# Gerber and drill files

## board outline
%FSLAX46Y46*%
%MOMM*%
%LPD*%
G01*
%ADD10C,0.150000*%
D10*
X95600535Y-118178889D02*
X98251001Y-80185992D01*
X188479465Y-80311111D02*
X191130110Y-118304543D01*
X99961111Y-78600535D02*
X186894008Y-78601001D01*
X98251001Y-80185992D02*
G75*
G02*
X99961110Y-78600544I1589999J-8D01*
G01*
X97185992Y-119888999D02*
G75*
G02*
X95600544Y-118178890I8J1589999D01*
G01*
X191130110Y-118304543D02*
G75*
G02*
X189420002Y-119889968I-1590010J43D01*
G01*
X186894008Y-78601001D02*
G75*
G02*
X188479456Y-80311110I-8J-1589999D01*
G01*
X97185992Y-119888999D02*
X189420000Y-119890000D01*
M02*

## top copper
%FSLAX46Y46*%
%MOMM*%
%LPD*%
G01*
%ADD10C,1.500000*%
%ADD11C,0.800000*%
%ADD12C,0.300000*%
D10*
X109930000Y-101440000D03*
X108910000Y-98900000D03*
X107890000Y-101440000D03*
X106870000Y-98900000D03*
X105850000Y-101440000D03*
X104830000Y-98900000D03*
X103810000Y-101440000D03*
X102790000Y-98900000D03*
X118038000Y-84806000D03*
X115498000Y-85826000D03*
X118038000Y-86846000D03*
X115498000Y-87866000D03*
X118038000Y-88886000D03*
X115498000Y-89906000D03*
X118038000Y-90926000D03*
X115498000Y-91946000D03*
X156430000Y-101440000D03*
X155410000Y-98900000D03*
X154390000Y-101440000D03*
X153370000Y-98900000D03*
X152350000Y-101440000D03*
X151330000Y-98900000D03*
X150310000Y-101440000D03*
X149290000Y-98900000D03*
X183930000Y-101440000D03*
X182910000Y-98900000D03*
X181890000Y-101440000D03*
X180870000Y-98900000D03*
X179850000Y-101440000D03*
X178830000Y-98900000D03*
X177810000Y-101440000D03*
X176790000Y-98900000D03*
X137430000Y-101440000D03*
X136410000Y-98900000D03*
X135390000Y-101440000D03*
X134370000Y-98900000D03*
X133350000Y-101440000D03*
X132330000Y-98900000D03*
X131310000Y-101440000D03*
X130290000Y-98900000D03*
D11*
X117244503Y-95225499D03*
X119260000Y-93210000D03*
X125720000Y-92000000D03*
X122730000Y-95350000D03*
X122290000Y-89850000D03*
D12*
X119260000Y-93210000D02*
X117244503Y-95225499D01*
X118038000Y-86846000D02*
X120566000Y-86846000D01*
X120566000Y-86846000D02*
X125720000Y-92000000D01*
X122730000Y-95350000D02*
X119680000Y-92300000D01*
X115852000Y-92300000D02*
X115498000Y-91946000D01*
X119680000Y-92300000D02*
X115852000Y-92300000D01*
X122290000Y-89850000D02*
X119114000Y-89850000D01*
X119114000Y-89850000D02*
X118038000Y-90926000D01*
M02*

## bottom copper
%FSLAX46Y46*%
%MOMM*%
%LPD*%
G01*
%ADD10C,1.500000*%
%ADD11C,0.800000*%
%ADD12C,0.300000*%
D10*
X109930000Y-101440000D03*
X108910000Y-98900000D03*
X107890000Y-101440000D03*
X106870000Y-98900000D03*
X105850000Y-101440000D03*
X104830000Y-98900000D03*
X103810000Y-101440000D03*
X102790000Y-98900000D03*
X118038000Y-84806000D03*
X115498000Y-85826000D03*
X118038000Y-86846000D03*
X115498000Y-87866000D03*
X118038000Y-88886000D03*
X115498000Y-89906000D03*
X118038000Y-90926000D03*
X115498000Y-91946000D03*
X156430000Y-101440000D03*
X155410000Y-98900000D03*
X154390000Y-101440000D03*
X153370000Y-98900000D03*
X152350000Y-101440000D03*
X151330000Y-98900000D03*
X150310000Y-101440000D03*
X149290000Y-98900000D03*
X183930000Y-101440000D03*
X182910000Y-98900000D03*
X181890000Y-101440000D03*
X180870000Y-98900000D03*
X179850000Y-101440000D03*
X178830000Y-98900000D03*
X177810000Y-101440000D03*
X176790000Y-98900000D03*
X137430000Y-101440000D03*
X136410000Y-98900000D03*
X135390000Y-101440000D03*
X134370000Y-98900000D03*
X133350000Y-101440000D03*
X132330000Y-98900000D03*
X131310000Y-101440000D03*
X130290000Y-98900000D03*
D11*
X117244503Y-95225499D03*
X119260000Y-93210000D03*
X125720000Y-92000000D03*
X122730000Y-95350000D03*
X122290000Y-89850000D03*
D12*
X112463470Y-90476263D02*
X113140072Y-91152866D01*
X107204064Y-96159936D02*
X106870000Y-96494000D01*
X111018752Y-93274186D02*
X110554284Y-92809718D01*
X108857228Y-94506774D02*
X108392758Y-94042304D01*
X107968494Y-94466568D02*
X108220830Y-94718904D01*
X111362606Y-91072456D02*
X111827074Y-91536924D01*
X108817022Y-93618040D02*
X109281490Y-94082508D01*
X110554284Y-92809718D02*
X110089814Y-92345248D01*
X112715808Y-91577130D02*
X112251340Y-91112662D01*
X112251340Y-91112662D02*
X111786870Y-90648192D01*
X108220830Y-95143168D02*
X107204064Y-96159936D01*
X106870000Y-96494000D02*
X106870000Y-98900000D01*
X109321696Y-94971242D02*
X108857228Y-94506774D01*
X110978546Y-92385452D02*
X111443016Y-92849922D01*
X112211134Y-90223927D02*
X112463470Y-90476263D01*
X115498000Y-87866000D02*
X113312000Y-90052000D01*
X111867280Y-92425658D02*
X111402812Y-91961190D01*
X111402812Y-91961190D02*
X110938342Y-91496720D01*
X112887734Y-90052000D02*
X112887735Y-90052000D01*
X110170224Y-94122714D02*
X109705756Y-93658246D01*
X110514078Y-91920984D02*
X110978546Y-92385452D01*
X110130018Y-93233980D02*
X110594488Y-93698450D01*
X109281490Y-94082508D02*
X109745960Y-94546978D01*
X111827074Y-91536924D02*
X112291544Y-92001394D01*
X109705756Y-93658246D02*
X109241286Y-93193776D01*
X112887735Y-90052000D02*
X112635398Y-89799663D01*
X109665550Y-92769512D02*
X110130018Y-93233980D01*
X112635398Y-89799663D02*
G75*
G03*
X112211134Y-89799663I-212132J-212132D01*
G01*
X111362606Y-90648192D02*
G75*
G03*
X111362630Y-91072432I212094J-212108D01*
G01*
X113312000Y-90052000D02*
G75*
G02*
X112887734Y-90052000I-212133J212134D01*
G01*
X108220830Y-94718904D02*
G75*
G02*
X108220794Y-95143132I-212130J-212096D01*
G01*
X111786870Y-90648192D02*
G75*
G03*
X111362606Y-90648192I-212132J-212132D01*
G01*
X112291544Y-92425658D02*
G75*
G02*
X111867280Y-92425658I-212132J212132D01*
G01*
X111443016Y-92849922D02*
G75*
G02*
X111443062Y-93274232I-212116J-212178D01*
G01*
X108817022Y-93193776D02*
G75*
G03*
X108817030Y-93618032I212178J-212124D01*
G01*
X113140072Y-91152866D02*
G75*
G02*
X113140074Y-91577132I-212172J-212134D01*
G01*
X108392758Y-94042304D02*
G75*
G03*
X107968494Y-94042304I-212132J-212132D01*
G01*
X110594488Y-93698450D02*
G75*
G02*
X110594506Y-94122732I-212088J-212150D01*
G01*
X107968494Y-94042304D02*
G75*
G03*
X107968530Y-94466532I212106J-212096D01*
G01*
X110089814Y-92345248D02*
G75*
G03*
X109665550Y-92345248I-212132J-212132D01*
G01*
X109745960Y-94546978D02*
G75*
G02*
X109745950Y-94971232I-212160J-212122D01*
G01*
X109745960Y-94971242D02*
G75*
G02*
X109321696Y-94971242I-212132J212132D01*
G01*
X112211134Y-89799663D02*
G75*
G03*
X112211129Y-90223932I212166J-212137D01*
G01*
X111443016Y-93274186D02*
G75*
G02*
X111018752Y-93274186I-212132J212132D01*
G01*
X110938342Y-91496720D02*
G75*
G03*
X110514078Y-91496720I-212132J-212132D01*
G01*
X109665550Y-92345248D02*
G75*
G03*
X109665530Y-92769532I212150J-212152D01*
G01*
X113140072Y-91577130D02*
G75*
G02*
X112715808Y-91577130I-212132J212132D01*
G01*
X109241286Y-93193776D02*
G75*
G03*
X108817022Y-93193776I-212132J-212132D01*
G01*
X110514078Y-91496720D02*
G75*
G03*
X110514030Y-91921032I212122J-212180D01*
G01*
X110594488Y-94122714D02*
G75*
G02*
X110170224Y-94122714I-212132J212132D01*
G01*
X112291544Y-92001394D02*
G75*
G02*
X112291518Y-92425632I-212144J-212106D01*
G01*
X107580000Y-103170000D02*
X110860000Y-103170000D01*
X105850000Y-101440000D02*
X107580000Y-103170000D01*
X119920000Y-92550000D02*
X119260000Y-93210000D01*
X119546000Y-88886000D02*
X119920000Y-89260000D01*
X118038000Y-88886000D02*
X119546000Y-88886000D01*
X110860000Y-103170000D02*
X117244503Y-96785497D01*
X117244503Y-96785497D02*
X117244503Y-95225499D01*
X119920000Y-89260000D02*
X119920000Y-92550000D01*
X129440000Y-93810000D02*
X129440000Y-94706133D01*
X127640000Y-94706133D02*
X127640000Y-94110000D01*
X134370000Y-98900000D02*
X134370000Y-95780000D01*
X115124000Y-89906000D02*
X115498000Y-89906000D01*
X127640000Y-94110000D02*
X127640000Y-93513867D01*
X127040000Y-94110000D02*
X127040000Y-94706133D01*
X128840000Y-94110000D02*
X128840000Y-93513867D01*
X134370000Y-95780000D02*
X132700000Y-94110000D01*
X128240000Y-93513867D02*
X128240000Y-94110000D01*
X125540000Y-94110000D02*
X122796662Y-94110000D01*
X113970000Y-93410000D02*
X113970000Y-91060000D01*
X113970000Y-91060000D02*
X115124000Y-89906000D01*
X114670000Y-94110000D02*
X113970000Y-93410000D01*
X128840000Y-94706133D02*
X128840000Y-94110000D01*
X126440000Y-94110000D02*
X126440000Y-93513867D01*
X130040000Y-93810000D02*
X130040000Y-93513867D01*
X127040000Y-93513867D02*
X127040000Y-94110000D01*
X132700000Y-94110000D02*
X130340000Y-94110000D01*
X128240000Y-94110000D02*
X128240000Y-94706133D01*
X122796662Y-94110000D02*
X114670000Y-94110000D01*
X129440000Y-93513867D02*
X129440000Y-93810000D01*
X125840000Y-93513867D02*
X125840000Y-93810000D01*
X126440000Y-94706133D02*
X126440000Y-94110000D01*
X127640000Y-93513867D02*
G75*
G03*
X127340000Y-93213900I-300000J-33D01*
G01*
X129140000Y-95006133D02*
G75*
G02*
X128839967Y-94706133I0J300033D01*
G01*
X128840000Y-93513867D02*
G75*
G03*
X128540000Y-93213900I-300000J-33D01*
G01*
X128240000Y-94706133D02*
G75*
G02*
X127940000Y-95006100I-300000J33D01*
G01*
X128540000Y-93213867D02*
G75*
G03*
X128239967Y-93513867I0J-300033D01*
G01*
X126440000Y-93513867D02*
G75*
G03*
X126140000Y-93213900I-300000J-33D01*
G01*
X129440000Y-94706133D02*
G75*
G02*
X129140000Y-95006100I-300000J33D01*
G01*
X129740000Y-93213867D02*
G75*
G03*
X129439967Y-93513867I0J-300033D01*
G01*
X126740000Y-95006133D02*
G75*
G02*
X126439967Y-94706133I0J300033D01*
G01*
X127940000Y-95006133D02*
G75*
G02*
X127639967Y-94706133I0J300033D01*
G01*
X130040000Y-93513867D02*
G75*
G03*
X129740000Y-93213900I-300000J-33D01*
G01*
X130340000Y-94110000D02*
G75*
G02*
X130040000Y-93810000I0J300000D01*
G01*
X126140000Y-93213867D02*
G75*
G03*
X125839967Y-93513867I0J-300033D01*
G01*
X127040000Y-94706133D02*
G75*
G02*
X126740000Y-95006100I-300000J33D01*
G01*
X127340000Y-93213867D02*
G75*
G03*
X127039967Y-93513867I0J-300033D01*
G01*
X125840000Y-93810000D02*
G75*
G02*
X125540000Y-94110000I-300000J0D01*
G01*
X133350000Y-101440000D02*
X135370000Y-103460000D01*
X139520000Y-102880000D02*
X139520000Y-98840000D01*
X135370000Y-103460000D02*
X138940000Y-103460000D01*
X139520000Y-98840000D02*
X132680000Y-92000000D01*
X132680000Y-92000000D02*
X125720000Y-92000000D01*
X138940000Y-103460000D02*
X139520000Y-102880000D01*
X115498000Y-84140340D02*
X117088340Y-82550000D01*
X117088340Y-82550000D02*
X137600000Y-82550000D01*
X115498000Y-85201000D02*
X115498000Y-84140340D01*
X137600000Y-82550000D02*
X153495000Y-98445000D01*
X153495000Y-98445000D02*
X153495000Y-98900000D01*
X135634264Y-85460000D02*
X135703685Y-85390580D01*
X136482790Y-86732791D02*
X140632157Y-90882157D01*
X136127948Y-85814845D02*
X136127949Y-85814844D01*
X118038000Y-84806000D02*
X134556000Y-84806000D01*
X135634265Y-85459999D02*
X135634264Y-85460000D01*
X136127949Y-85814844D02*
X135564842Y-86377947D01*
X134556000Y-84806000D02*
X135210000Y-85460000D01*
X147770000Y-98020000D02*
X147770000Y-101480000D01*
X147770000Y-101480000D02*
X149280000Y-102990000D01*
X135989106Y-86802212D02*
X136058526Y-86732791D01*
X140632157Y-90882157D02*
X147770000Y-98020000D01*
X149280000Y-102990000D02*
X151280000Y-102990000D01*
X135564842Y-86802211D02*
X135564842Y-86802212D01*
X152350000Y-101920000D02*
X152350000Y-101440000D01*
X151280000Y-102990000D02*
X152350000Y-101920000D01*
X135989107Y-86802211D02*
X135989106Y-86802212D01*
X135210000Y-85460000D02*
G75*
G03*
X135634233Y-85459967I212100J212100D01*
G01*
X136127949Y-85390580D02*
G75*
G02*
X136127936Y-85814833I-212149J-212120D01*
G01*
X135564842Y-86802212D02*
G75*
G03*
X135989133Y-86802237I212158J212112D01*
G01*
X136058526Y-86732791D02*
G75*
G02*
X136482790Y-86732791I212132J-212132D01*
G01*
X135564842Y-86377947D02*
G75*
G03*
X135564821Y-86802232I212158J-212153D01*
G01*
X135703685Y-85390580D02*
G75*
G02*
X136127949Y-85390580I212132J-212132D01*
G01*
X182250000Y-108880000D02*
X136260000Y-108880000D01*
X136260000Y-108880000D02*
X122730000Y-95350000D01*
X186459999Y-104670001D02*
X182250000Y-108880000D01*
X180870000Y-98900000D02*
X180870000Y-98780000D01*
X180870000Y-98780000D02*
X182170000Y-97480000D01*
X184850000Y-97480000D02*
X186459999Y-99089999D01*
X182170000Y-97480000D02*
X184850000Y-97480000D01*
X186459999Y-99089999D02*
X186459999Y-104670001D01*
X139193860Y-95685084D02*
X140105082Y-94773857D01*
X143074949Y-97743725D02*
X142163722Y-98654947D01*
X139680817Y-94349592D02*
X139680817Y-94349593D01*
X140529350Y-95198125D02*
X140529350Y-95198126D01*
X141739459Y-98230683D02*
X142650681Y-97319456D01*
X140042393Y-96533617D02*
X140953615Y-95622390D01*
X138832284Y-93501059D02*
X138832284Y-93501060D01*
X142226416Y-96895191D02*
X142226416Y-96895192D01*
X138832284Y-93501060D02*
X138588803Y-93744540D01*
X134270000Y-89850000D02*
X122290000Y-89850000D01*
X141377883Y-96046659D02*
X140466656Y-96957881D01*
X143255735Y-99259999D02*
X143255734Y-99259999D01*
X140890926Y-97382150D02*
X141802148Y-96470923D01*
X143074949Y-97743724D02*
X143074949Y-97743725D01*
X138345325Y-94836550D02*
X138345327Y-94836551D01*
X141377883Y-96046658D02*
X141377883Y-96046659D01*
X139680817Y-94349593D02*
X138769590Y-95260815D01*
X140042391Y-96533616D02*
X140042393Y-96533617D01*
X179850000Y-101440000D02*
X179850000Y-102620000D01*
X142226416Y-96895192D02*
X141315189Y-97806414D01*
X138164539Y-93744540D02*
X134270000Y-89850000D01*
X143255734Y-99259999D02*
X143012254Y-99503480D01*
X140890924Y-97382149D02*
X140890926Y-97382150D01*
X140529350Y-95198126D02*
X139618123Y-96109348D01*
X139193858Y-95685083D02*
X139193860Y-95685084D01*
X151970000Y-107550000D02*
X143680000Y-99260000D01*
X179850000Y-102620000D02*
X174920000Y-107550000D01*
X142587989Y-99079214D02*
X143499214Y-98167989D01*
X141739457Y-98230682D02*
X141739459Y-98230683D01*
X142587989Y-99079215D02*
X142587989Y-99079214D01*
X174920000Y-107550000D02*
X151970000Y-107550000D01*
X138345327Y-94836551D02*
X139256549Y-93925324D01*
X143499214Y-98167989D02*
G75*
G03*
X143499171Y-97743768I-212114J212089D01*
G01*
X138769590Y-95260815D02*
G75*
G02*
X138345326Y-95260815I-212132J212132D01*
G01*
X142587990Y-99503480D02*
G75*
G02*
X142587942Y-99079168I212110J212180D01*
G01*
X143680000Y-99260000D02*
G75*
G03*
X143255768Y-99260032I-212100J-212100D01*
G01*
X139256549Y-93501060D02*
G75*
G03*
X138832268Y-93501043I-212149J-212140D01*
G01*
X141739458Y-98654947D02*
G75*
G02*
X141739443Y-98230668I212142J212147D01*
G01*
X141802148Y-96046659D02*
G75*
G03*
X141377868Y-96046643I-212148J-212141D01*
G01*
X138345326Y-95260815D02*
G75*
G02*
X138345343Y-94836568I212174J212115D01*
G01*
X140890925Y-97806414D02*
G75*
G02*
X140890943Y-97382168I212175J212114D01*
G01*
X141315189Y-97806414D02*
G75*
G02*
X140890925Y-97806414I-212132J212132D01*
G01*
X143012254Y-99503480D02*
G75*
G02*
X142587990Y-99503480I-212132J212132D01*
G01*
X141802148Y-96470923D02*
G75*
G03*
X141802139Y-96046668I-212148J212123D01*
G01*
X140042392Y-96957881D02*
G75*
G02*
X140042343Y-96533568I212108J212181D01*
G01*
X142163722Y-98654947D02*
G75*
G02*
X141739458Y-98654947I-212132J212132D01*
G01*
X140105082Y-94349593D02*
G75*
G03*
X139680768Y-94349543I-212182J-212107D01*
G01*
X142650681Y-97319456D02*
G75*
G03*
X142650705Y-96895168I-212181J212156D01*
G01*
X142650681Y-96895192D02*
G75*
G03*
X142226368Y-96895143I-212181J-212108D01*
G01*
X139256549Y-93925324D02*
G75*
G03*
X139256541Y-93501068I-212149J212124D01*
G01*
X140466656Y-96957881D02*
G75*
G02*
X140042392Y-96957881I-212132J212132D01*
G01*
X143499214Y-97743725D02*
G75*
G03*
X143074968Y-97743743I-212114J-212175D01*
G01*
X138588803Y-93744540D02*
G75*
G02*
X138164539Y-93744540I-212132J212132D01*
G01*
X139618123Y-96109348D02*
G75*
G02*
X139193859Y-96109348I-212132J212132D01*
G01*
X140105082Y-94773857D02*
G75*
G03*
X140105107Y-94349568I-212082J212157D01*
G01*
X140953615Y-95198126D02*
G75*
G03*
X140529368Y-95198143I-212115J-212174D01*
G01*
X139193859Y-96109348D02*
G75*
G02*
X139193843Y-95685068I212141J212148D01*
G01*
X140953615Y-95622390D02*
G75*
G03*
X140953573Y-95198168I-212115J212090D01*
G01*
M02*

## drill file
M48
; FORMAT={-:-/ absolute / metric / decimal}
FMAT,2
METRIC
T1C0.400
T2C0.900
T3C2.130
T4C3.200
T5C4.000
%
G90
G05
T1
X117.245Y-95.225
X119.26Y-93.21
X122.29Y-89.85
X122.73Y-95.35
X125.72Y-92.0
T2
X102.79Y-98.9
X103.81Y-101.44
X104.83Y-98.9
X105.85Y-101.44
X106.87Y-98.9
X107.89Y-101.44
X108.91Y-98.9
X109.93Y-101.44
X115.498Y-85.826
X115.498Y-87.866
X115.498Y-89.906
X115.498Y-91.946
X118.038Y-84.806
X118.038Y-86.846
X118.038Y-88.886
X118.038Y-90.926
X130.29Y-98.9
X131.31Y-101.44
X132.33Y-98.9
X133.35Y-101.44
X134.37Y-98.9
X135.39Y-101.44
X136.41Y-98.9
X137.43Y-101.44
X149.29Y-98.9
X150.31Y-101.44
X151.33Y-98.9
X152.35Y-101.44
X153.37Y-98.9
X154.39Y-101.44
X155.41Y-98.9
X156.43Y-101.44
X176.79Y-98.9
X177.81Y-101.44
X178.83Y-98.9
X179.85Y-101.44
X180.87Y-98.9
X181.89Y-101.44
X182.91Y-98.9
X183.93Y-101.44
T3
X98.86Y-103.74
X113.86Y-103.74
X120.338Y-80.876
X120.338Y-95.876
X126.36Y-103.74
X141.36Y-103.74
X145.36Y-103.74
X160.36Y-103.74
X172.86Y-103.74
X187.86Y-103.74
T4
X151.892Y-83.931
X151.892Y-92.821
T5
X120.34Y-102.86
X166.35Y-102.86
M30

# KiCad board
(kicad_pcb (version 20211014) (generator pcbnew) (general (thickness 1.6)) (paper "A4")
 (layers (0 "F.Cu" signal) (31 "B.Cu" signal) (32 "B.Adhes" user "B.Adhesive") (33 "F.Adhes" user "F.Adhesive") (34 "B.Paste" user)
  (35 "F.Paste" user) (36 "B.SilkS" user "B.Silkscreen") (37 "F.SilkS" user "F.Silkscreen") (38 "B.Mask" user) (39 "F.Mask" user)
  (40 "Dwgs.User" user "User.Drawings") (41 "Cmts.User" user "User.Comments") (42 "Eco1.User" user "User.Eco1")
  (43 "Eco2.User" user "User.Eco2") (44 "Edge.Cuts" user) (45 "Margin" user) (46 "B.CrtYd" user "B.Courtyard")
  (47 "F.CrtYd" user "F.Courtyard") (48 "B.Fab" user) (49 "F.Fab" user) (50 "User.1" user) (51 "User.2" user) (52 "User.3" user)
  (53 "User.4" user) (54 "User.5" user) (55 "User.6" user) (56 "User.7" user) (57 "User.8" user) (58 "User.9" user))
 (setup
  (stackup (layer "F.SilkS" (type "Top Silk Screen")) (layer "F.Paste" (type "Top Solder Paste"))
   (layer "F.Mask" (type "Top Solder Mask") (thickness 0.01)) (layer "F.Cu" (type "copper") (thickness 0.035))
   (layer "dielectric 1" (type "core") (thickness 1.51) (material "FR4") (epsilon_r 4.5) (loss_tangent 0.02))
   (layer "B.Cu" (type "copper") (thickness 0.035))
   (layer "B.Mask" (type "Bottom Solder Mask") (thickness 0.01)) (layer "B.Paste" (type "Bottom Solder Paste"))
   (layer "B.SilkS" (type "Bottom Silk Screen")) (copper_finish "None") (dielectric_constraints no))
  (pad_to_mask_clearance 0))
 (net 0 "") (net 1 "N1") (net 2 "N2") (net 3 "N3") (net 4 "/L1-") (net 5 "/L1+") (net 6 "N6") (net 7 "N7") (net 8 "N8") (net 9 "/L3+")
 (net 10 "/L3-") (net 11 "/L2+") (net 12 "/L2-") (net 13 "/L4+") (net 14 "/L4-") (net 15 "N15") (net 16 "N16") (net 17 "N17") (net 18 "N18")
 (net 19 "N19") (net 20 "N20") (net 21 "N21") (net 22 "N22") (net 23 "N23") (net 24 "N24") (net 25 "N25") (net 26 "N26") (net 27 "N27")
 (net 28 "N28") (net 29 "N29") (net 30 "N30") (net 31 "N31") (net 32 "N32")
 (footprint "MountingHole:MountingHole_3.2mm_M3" (layer "F.Cu") (at 151.892 83.931)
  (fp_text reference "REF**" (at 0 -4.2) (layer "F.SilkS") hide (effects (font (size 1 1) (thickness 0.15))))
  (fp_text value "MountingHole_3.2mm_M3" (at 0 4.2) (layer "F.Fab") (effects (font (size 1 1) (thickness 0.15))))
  (pad "" np_thru_hole circle (at 0 0) (size 3.2 3.2) (drill 3.2) (layers F&B.Cu *.Mask)))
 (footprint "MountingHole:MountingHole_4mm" (layer "F.Cu") (at 166.35 102.86)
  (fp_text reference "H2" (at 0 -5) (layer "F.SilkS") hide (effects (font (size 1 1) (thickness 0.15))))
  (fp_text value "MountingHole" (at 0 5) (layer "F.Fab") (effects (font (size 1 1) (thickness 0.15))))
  (pad "" np_thru_hole circle (at 0 0) (size 4 4) (drill 4) (layers *.Cu *.Mask)))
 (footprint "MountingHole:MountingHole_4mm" (layer "F.Cu") (at 120.34 102.86)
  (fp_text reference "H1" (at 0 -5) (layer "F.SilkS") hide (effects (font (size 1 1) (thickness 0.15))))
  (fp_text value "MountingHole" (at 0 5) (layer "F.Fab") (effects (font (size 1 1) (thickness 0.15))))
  (pad "" np_thru_hole circle (at 0 0) (size 4 4) (drill 4) (layers *.Cu *.Mask)))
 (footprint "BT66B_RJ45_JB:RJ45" (layer "F.Cu") (at 106.36 100.17)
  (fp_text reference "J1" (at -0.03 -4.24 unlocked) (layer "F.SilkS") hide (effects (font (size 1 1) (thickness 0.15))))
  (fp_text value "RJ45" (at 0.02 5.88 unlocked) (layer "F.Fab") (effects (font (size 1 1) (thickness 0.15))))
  (pad "" np_thru_hole circle (at -7.5 3.57) (size 2.13 2.13) (drill 2.13) (layers F&B.Cu *.SilkS *.Mask))
  (pad "" np_thru_hole circle (at 7.5 3.57) (size 2.13 2.13) (drill 2.13) (layers F&B.Cu *.SilkS *.Mask))
  (pad "1" thru_hole circle (at 3.57 1.27 180) (size 1.5 1.5) (drill 0.9) (layers *.Cu *.Mask) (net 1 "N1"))
  (pad "2" thru_hole circle (at 2.55 -1.27 180) (size 1.5 1.5) (drill 0.9) (layers *.Cu *.Mask) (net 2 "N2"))
  (pad "3" thru_hole circle (at 1.53 1.27 180) (size 1.5 1.5) (drill 0.9) (layers *.Cu *.Mask) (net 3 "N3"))
  (pad "4" thru_hole circle (at 0.51 -1.27 180) (size 1.5 1.5) (drill 0.9) (layers *.Cu *.Mask) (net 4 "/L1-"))
  (pad "5" thru_hole circle (at -0.51 1.27 180) (size 1.5 1.5) (drill 0.9) (layers *.Cu *.Mask) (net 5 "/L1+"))
  (pad "6" thru_hole circle (at -1.53 -1.27 180) (size 1.5 1.5) (drill 0.9) (layers *.Cu *.Mask) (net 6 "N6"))
  (pad "7" thru_hole circle (at -2.55 1.27 180) (size 1.5 1.5) (drill 0.9) (layers *.Cu *.Mask) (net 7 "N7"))
  (pad "8" thru_hole circle (at -3.57 -1.27 180) (size 1.5 1.5) (drill 0.9) (layers *.Cu *.Mask) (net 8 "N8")))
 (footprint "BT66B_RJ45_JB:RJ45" (layer "F.Cu") (at 116.768 88.376 90)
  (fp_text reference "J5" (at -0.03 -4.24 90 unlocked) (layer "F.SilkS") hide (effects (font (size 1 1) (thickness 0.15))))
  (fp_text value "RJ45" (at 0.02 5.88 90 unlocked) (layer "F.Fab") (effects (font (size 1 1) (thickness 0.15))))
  (pad "" np_thru_hole circle (at 7.5 3.57 90) (size 2.13 2.13) (drill 2.13) (layers F&B.Cu *.SilkS *.Mask))
  (pad "" np_thru_hole circle (at -7.5 3.57 90) (size 2.13 2.13) (drill 2.13) (layers F&B.Cu *.SilkS *.Mask))
  (pad "1" thru_hole circle (at 3.57 1.27 270) (size 1.5 1.5) (drill 0.9) (layers *.Cu *.Mask) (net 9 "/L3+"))
  (pad "2" thru_hole circle (at 2.55 -1.27 270) (size 1.5 1.5) (drill 0.9) (layers *.Cu *.Mask) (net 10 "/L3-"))
  (pad "3" thru_hole circle (at 1.53 1.27 270) (size 1.5 1.5) (drill 0.9) (layers *.Cu *.Mask) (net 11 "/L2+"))
  (pad "4" thru_hole circle (at 0.51 -1.27 270) (size 1.5 1.5) (drill 0.9) (layers *.Cu *.Mask) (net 4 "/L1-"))
  (pad "5" thru_hole circle (at -0.51 1.27 270) (size 1.5 1.5) (drill 0.9) (layers *.Cu *.Mask) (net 5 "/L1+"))
  (pad "6" thru_hole circle (at -1.53 -1.27 270) (size 1.5 1.5) (drill 0.9) (layers *.Cu *.Mask) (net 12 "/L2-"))
  (pad "7" thru_hole circle (at -2.55 1.27 270) (size 1.5 1.5) (drill 0.9) (layers *.Cu *.Mask) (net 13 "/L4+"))
  (pad "8" thru_hole circle (at -3.57 -1.27 270) (size 1.5 1.5) (drill 0.9) (layers *.Cu *.Mask) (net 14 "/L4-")))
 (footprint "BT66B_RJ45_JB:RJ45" (layer "F.Cu") (at 152.86 100.17)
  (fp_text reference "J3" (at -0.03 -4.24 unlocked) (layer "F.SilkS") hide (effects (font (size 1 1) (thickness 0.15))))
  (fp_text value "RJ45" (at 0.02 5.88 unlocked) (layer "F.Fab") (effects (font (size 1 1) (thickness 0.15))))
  (pad "" np_thru_hole circle (at -7.5 3.57) (size 2.13 2.13) (drill 2.13) (layers F&B.Cu *.SilkS *.Mask))
  (pad "" np_thru_hole circle (at 7.5 3.57) (size 2.13 2.13) (drill 2.13) (layers F&B.Cu *.SilkS *.Mask))
  (pad "1" thru_hole circle (at 3.57 1.27 180) (size 1.5 1.5) (drill 0.9) (layers *.Cu *.Mask) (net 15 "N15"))
  (pad "2" thru_hole circle (at 2.55 -1.27 180) (size 1.5 1.5) (drill 0.9) (layers *.Cu *.Mask) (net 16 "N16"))
  (pad "3" thru_hole circle (at 1.53 1.27 180) (size 1.5 1.5) (drill 0.9) (layers *.Cu *.Mask) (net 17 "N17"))
  (pad "4" thru_hole circle (at 0.51 -1.27 180) (size 1.5 1.5) (drill 0.9) (layers *.Cu *.Mask) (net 10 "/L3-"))
  (pad "5" thru_hole circle (at -0.51 1.27 180) (size 1.5 1.5) (drill 0.9) (layers *.Cu *.Mask) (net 9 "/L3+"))
  (pad "6" thru_hole circle (at -1.53 -1.27 180) (size 1.5 1.5) (drill 0.9) (layers *.Cu *.Mask) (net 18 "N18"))
  (pad "7" thru_hole circle (at -2.55 1.27 180) (size 1.5 1.5) (drill 0.9) (layers *.Cu *.Mask) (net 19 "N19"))
  (pad "8" thru_hole circle (at -3.57 -1.27 180) (size 1.5 1.5) (drill 0.9) (layers *.Cu *.Mask) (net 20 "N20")))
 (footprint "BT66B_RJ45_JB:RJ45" (layer "F.Cu") (at 180.36 100.17)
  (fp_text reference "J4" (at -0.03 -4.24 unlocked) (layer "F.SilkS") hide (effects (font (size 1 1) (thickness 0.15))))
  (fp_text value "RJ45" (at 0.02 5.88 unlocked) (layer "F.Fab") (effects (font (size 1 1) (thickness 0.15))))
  (pad "" np_thru_hole circle (at 7.5 3.57) (size 2.13 2.13) (drill 2.13) (layers F&B.Cu *.SilkS *.Mask))
  (pad "" np_thru_hole circle (at -7.5 3.57) (size 2.13 2.13) (drill 2.13) (layers F&B.Cu *.SilkS *.Mask))
  (pad "1" thru_hole circle (at 3.57 1.27 180) (size 1.5 1.5) (drill 0.9) (layers *.Cu *.Mask) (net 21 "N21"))
  (pad "2" thru_hole circle (at 2.55 -1.27 180) (size 1.5 1.5) (drill 0.9) (layers *.Cu *.Mask) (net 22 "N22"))
  (pad "3" thru_hole circle (at 1.53 1.27 180) (size 1.5 1.5) (drill 0.9) (layers *.Cu *.Mask) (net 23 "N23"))
  (pad "4" thru_hole circle (at 0.51 -1.27 180) (size 1.5 1.5) (drill 0.9) (layers *.Cu *.Mask) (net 14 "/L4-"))
  (pad "5" thru_hole circle (at -0.51 1.27 180) (size 1.5 1.5) (drill 0.9) (layers *.Cu *.Mask) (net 13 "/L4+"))
  (pad "6" thru_hole circle (at -1.53 -1.27 180) (size 1.5 1.5) (drill 0.9) (layers *.Cu *.Mask) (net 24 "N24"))
  (pad "7" thru_hole circle (at -2.55 1.27 180) (size 1.5 1.5) (drill 0.9) (layers *.Cu *.Mask) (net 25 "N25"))
  (pad "8" thru_hole circle (at -3.57 -1.27 180) (size 1.5 1.5) (drill 0.9) (layers *.Cu *.Mask) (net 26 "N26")))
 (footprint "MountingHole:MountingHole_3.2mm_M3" (layer "F.Cu") (at 151.892 92.821)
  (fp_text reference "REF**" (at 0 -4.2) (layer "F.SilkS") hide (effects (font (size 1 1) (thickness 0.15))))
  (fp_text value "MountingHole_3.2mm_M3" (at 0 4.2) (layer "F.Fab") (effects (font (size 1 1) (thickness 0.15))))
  (pad "" np_thru_hole circle (at 0 0) (size 3.2 3.2) (drill 3.2) (layers F&B.Cu *.Mask)))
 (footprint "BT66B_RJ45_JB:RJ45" (layer "F.Cu") (at 133.86 100.17)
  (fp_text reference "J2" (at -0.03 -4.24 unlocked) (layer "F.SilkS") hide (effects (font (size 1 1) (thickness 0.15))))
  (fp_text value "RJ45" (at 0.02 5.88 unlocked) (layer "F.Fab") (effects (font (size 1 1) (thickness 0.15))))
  (pad "" np_thru_hole circle (at -7.5 3.57) (size 2.13 2.13) (drill 2.13) (layers F&B.Cu *.SilkS *.Mask))
  (pad "" np_thru_hole circle (at 7.5 3.57) (size 2.13 2.13) (drill 2.13) (layers F&B.Cu *.SilkS *.Mask))
  (pad "1" thru_hole circle (at 3.57 1.27 180) (size 1.5 1.5) (drill 0.9) (layers *.Cu *.Mask) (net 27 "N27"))
  (pad "2" thru_hole circle (at 2.55 -1.27 180) (size 1.5 1.5) (drill 0.9) (layers *.Cu *.Mask) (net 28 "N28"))
  (pad "3" thru_hole circle (at 1.53 1.27 180) (size 1.5 1.5) (drill 0.9) (layers *.Cu *.Mask) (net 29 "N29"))
  (pad "4" thru_hole circle (at 0.51 -1.27 180) (size 1.5 1.5) (drill 0.9) (layers *.Cu *.Mask) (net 12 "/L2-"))
  (pad "5" thru_hole circle (at -0.51 1.27 180) (size 1.5 1.5) (drill 0.9) (layers *.Cu *.Mask) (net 11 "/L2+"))
  (pad "6" thru_hole circle (at -1.53 -1.27 180) (size 1.5 1.5) (drill 0.9) (layers *.Cu *.Mask) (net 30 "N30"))
  (pad "7" thru_hole circle (at -2.55 1.27 180) (size 1.5 1.5) (drill 0.9) (layers *.Cu *.Mask) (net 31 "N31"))
  (pad "8" thru_hole circle (at -3.57 -1.27 180) (size 1.5 1.5) (drill 0.9) (layers *.Cu *.Mask) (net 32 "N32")))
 (gr_line (start 95.600535 118.178889) (end 98.251001 80.185992) (layer "Edge.Cuts") (width 0.15))
 (gr_line (start 188.479465 80.311111) (end 191.13011 118.304543) (layer "Edge.Cuts") (width 0.15))
 (gr_line (start 99.961111 78.600535) (end 186.894008 78.601001) (layer "Edge.Cuts") (width 0.15))
 (gr_arc (start 98.251001 80.185992) (mid 98.76 79.02) (end 99.961111 78.600535) (layer "Edge.Cuts") (width 0.15))
 (gr_arc (start 97.185992 119.888999) (mid 96.02 119.38) (end 95.600535 118.178889) (layer "Edge.Cuts") (width 0.15))
 (gr_arc (start 191.13011 118.304543) (mid 190.621111 119.470535) (end 189.42 119.89) (layer "Edge.Cuts") (width 0.15))
 (gr_arc (start 186.894008 78.601001) (mid 188.06 79.11) (end 188.479465 80.311111) (layer "Edge.Cuts") (width 0.15))
 (gr_line (start 97.185992 119.888999) (end 189.42 119.89) (layer "Edge.Cuts") (width 0.15))
 (segment (start 112.46347 90.476263) (end 113.140072 91.152866) (width 0.3) (layer "B.Cu") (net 4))
 (segment (start 107.204064 96.159936) (end 106.87 96.494) (width 0.3) (layer "B.Cu") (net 4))
 (segment (start 111.018752 93.274186) (end 110.554284 92.809718) (width 0.3) (layer "B.Cu") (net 4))
 (segment (start 108.857228 94.506774) (end 108.392758 94.042304) (width 0.3) (layer "B.Cu") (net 4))
 (segment (start 107.968494 94.466568) (end 108.22083 94.718904) (width 0.3) (layer "B.Cu") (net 4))
 (segment (start 111.362606 91.072456) (end 111.827074 91.536924) (width 0.3) (layer "B.Cu") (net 4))
 (segment (start 108.817022 93.61804) (end 109.28149 94.082508) (width 0.3) (layer "B.Cu") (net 4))
 (segment (start 110.554284 92.809718) (end 110.089814 92.345248) (width 0.3) (layer "B.Cu") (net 4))
 (segment (start 112.715808 91.57713) (end 112.25134 91.112662) (width 0.3) (layer "B.Cu") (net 4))
 (segment (start 112.25134 91.112662) (end 111.78687 90.648192) (width 0.3) (layer "B.Cu") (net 4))
 (segment (start 108.22083 95.143168) (end 107.204064 96.159936) (width 0.3) (layer "B.Cu") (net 4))
 (segment (start 106.87 96.494) (end 106.87 98.9) (width 0.3) (layer "B.Cu") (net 4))
 (segment (start 109.321696 94.971242) (end 108.857228 94.506774) (width 0.3) (layer "B.Cu") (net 4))
 (segment (start 110.978546 92.385452) (end 111.443016 92.849922) (width 0.3) (layer "B.Cu") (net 4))
 (segment (start 112.211134 90.223927) (end 112.46347 90.476263) (width 0.3) (layer "B.Cu") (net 4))
 (segment (start 115.498 87.866) (end 113.312 90.052) (width 0.3) (layer "B.Cu") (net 4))
 (segment (start 111.86728 92.425658) (end 111.402812 91.96119) (width 0.3) (layer "B.Cu") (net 4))
 (segment (start 111.402812 91.96119) (end 110.938342 91.49672) (width 0.3) (layer "B.Cu") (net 4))
 (segment (start 112.887734 90.052) (end 112.887735 90.052) (width 0.3) (layer "B.Cu") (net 4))
 (segment (start 110.170224 94.122714) (end 109.705756 93.658246) (width 0.3) (layer "B.Cu") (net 4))
 (segment (start 110.514078 91.920984) (end 110.978546 92.385452) (width 0.3) (layer "B.Cu") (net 4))
 (segment (start 110.130018 93.23398) (end 110.594488 93.69845) (width 0.3) (layer "B.Cu") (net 4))
 (segment (start 109.28149 94.082508) (end 109.74596 94.546978) (width 0.3) (layer "B.Cu") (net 4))
 (segment (start 111.827074 91.536924) (end 112.291544 92.001394) (width 0.3) (layer "B.Cu") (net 4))
 (segment (start 109.705756 93.658246) (end 109.241286 93.193776) (width 0.3) (layer "B.Cu") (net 4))
 (segment (start 112.887735 90.052) (end 112.635398 89.799663) (width 0.3) (layer "B.Cu") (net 4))
 (segment (start 109.66555 92.769512) (end 110.130018 93.23398) (width 0.3) (layer "B.Cu") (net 4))
 (arc (start 112.635398 89.799663) (mid 112.423266 89.711795) (end 112.211134 89.799663) (width 0.3) (layer "B.Cu") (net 4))
 (arc (start 111.362606 90.648192) (mid 111.274738 90.860324) (end 111.362606 91.072456) (width 0.3) (layer "B.Cu") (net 4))
 (arc (start 113.312 90.052) (mid 113.099867 90.139868) (end 112.887734 90.052) (width 0.3) (layer "B.Cu") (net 4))
 (arc (start 108.22083 94.718904) (mid 108.308698 94.931036) (end 108.22083 95.143168) (width 0.3) (layer "B.Cu") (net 4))
 (arc (start 111.78687 90.648192) (mid 111.574738 90.560324) (end 111.362606 90.648192) (width 0.3) (layer "B.Cu") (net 4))
 (arc (start 112.291544 92.425658) (mid 112.079412 92.513526) (end 111.86728 92.425658) (width 0.3) (layer "B.Cu") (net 4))
 (arc (start 111.443016 92.849922) (mid 111.530884 93.062054) (end 111.443016 93.274186) (width 0.3) (layer "B.Cu") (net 4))
 (arc (start 108.817022 93.193776) (mid 108.729154 93.405908) (end 108.817022 93.61804) (width 0.3) (layer "B.Cu") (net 4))
 (arc (start 113.140072 91.152866) (mid 113.22794 91.364998) (end 113.140072 91.57713) (width 0.3) (layer "B.Cu") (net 4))
 (arc (start 108.392758 94.042304) (mid 108.180626 93.954436) (end 107.968494 94.042304) (width 0.3) (layer "B.Cu") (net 4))
 (arc (start 110.594488 93.69845) (mid 110.682356 93.910582) (end 110.594488 94.122714) (width 0.3) (layer "B.Cu") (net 4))
 (arc (start 107.968494 94.042304) (mid 107.880626 94.254436) (end 107.968494 94.466568) (width 0.3) (layer "B.Cu") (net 4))
 (arc (start 110.089814 92.345248) (mid 109.877682 92.25738) (end 109.66555 92.345248) (width 0.3) (layer "B.Cu") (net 4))
 (arc (start 109.74596 94.546978) (mid 109.833828 94.75911) (end 109.74596 94.971242) (width 0.3) (layer "B.Cu") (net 4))
 (arc (start 109.74596 94.971242) (mid 109.533828 95.05911) (end 109.321696 94.971242) (width 0.3) (layer "B.Cu") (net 4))
 (arc (start 112.211134 89.799663) (mid 112.123266 90.011795) (end 112.211134 90.223927) (width 0.3) (layer "B.Cu") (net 4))
 (arc (start 111.443016 93.274186) (mid 111.230884 93.362054) (end 111.018752 93.274186) (width 0.3) (layer "B.Cu") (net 4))
 (arc (start 110.938342 91.49672) (mid 110.72621 91.408852) (end 110.514078 91.49672) (width 0.3) (layer "B.Cu") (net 4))
 (arc (start 109.66555 92.345248) (mid 109.577682 92.55738) (end 109.66555 92.769512) (width 0.3) (layer "B.Cu") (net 4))
 (arc (start 113.140072 91.57713) (mid 112.92794 91.664998) (end 112.715808 91.57713) (width 0.3) (layer "B.Cu") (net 4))
 (arc (start 109.241286 93.193776) (mid 109.029154 93.105908) (end 108.817022 93.193776) (width 0.3) (layer "B.Cu") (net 4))
 (arc (start 110.514078 91.49672) (mid 110.42621 91.708852) (end 110.514078 91.920984) (width 0.3) (layer "B.Cu") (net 4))
 (arc (start 110.594488 94.122714) (mid 110.382356 94.210582) (end 110.170224 94.122714) (width 0.3) (layer "B.Cu") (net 4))
 (arc (start 112.291544 92.001394) (mid 112.379412 92.213526) (end 112.291544 92.425658) (width 0.3) (layer "B.Cu") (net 4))
 (segment (start 119.26 93.21) (end 117.244503 95.225499) (width 0.3) (layer "F.Cu") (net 5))
 (via (at 117.244503 95.225499) (size 0.8) (drill 0.4) (layers "F.Cu" "B.Cu") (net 5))
 (via (at 119.26 93.21) (size 0.8) (drill 0.4) (layers "F.Cu" "B.Cu") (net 5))
 (segment (start 107.58 103.17) (end 110.86 103.17) (width 0.3) (layer "B.Cu") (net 5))
 (segment (start 105.85 101.44) (end 107.58 103.17) (width 0.3) (layer "B.Cu") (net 5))
 (segment (start 119.92 92.55) (end 119.26 93.21) (width 0.3) (layer "B.Cu") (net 5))
 (segment (start 119.546 88.886) (end 119.92 89.26) (width 0.3) (layer "B.Cu") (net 5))
 (segment (start 118.038 88.886) (end 119.546 88.886) (width 0.3) (layer "B.Cu") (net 5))
 (segment (start 110.86 103.17) (end 117.244503 96.785497) (width 0.3) (layer "B.Cu") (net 5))
 (segment (start 117.244503 96.785497) (end 117.244503 95.225499) (width 0.3) (layer "B.Cu") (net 5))
 (segment (start 119.92 89.26) (end 119.92 92.55) (width 0.3) (layer "B.Cu") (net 5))
 (segment (start 129.44 93.81) (end 129.44 94.706133) (width 0.3) (layer "B.Cu") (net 12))
 (segment (start 127.64 94.706133) (end 127.64 94.11) (width 0.3) (layer "B.Cu") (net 12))
 (segment (start 134.37 98.9) (end 134.37 95.78) (width 0.3) (layer "B.Cu") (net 12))
 (segment (start 115.124 89.906) (end 115.498 89.906) (width 0.3) (layer "B.Cu") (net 12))
 (segment (start 127.64 94.11) (end 127.64 93.513867) (width 0.3) (layer "B.Cu") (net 12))
 (segment (start 127.04 94.11) (end 127.04 94.706133) (width 0.3) (layer "B.Cu") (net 12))
 (segment (start 128.84 94.11) (end 128.84 93.513867) (width 0.3) (layer "B.Cu") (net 12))
 (segment (start 134.37 95.78) (end 132.7 94.11) (width 0.3) (layer "B.Cu") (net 12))
 (segment (start 128.24 93.513867) (end 128.24 94.11) (width 0.3) (layer "B.Cu") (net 12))
 (segment (start 125.54 94.11) (end 122.796662 94.11) (width 0.3) (layer "B.Cu") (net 12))
 (segment (start 113.97 93.41) (end 113.97 91.06) (width 0.3) (layer "B.Cu") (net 12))
 (segment (start 113.97 91.06) (end 115.124 89.906) (width 0.3) (layer "B.Cu") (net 12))
 (segment (start 114.67 94.11) (end 113.97 93.41) (width 0.3) (layer "B.Cu") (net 12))
 (segment (start 128.84 94.706133) (end 128.84 94.11) (width 0.3) (layer "B.Cu") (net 12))
 (segment (start 126.44 94.11) (end 126.44 93.513867) (width 0.3) (layer "B.Cu") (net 12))
 (segment (start 130.04 93.81) (end 130.04 93.513867) (width 0.3) (layer "B.Cu") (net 12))
 (segment (start 127.04 93.513867) (end 127.04 94.11) (width 0.3) (layer "B.Cu") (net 12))
 (segment (start 132.7 94.11) (end 130.34 94.11) (width 0.3) (layer "B.Cu") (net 12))
 (segment (start 128.24 94.11) (end 128.24 94.706133) (width 0.3) (layer "B.Cu") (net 12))
 (segment (start 122.796662 94.11) (end 114.67 94.11) (width 0.3) (layer "B.Cu") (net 12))
 (segment (start 129.44 93.513867) (end 129.44 93.81) (width 0.3) (layer "B.Cu") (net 12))
 (segment (start 125.84 93.513867) (end 125.84 93.81) (width 0.3) (layer "B.Cu") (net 12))
 (segment (start 126.44 94.706133) (end 126.44 94.11) (width 0.3) (layer "B.Cu") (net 12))
 (arc (start 127.64 93.513867) (mid 127.552132 93.301735) (end 127.34 93.213867) (width 0.3) (layer "B.Cu") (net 12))
 (arc (start 129.14 95.006133) (mid 128.927868 94.918265) (end 128.84 94.706133) (width 0.3) (layer "B.Cu") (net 12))
 (arc (start 128.84 93.513867) (mid 128.752132 93.301735) (end 128.54 93.213867) (width 0.3) (layer "B.Cu") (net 12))
 (arc (start 128.24 94.706133) (mid 128.152132 94.918265) (end 127.94 95.006133) (width 0.3) (layer "B.Cu") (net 12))
 (arc (start 128.54 93.213867) (mid 128.327868 93.301735) (end 128.24 93.513867) (width 0.3) (layer "B.Cu") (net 12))
 (arc (start 126.44 93.513867) (mid 126.352132 93.301735) (end 126.14 93.213867) (width 0.3) (layer "B.Cu") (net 12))
 (arc (start 129.44 94.706133) (mid 129.352132 94.918265) (end 129.14 95.006133) (width 0.3) (layer "B.Cu") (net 12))
 (arc (start 129.74 93.213867) (mid 129.527868 93.301735) (end 129.44 93.513867) (width 0.3) (layer "B.Cu") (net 12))
 (arc (start 126.74 95.006133) (mid 126.527868 94.918265) (end 126.44 94.706133) (width 0.3) (layer "B.Cu") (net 12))
 (arc (start 127.94 95.006133) (mid 127.727868 94.918265) (end 127.64 94.706133) (width 0.3) (layer "B.Cu") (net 12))
 (arc (start 130.04 93.513867) (mid 129.952132 93.301735) (end 129.74 93.213867) (width 0.3) (layer "B.Cu") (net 12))
 (arc (start 130.34 94.11) (mid 130.127868 94.022132) (end 130.04 93.81) (width 0.3) (layer "B.Cu") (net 12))
 (arc (start 126.14 93.213867) (mid 125.927868 93.301735) (end 125.84 93.513867) (width 0.3) (layer "B.Cu") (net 12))
 (arc (start 127.04 94.706133) (mid 126.952132 94.918265) (end 126.74 95.006133) (width 0.3) (layer "B.Cu") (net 12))
 (arc (start 127.34 93.213867) (mid 127.127868 93.301735) (end 127.04 93.513867) (width 0.3) (layer "B.Cu") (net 12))
 (arc (start 125.84 93.81) (mid 125.752132 94.022132) (end 125.54 94.11) (width 0.3) (layer "B.Cu") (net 12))
 (segment (start 118.038 86.846) (end 120.566 86.846) (width 0.3) (layer "F.Cu") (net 11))
 (segment (start 120.566 86.846) (end 125.72 92) (width 0.3) (layer "F.Cu") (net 11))
 (via (at 125.72 92) (size 0.8) (drill 0.4) (layers "F.Cu" "B.Cu") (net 11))
 (segment (start 133.35 101.44) (end 135.37 103.46) (width 0.3) (layer "B.Cu") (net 11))
 (segment (start 139.52 102.88) (end 139.52 98.84) (width 0.3) (layer "B.Cu") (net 11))
 (segment (start 135.37 103.46) (end 138.94 103.46) (width 0.3) (layer "B.Cu") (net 11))
 (segment (start 139.52 98.84) (end 132.68 92) (width 0.3) (layer "B.Cu") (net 11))
 (segment (start 132.68 92) (end 125.72 92) (width 0.3) (layer "B.Cu") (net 11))
 (segment (start 138.94 103.46) (end 139.52 102.88) (width 0.3) (layer "B.Cu") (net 11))
 (segment (start 115.498 84.14034) (end 117.08834 82.55) (width 0.3) (layer "B.Cu") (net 10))
 (segment (start 117.08834 82.55) (end 137.6 82.55) (width 0.3) (layer "B.Cu") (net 10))
 (segment (start 115.498 85.201) (end 115.498 84.14034) (width 0.3) (layer "B.Cu") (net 10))
 (segment (start 137.6 82.55) (end 153.495 98.445) (width 0.3) (layer "B.Cu") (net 10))
 (segment (start 153.495 98.445) (end 153.495 98.9) (width 0.3) (layer "B.Cu") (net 10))
 (segment (start 135.634264 85.46) (end 135.703685 85.39058) (width 0.3) (layer "B.Cu") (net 9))
 (segment (start 136.48279 86.732791) (end 140.632157 90.882157) (width 0.3) (layer "B.Cu") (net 9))
 (segment (start 136.127948 85.814845) (end 136.127949 85.814844) (width 0.3) (layer "B.Cu") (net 9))
 (segment (start 118.038 84.806) (end 134.556 84.806) (width 0.3) (layer "B.Cu") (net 9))
 (segment (start 135.634265 85.459999) (end 135.634264 85.46) (width 0.3) (layer "B.Cu") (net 9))
 (segment (start 136.127949 85.814844) (end 135.564842 86.377947) (width 0.3) (layer "B.Cu") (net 9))
 (segment (start 134.556 84.806) (end 135.21 85.46) (width 0.3) (layer "B.Cu") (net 9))
 (segment (start 147.77 98.02) (end 147.77 101.48) (width 0.3) (layer "B.Cu") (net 9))
 (segment (start 147.77 101.48) (end 149.28 102.99) (width 0.3) (layer "B.Cu") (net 9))
 (segment (start 135.989106 86.802212) (end 136.058526 86.732791) (width 0.3) (layer "B.Cu") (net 9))
 (segment (start 140.632157 90.882157) (end 147.77 98.02) (width 0.3) (layer "B.Cu") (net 9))
 (segment (start 149.28 102.99) (end 151.28 102.99) (width 0.3) (layer "B.Cu") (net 9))
 (segment (start 135.564842 86.802211) (end 135.564842 86.802212) (width 0.3) (layer "B.Cu") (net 9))
 (segment (start 152.35 101.92) (end 152.35 101.44) (width 0.3) (layer "B.Cu") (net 9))
 (segment (start 151.28 102.99) (end 152.35 101.92) (width 0.3) (layer "B.Cu") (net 9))
 (segment (start 135.989107 86.802211) (end 135.989106 86.802212) (width 0.3) (layer "B.Cu") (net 9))
 (arc (start 135.21 85.46) (mid 135.422134 85.547869) (end 135.634265 85.459999) (width 0.3) (layer "B.Cu") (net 9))
 (arc (start 136.127949 85.39058) (mid 136.215816 85.602712) (end 136.127948 85.814845) (width 0.3) (layer "B.Cu") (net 9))
 (arc (start 135.564842 86.802212) (mid 135.776975 86.89008) (end 135.989107 86.802211) (width 0.3) (layer "B.Cu") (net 9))
 (arc (start 136.058526 86.732791) (mid 136.270658 86.644923) (end 136.48279 86.732791) (width 0.3) (layer "B.Cu") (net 9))
 (arc (start 135.564842 86.377947) (mid 135.476974 86.590079) (end 135.564842 86.802211) (width 0.3) (layer "B.Cu") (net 9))
 (arc (start 135.703685 85.39058) (mid 135.915817 85.302712) (end 136.127949 85.39058) (width 0.3) (layer "B.Cu") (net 9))
 (segment (start 122.73 95.35) (end 119.68 92.3) (width 0.3) (layer "F.Cu") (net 14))
 (segment (start 115.852 92.3) (end 115.498 91.946) (width 0.3) (layer "F.Cu") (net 14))
 (segment (start 119.68 92.3) (end 115.852 92.3) (width 0.3) (layer "F.Cu") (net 14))
 (via (at 122.73 95.35) (size 0.8) (drill 0.4) (layers "F.Cu" "B.Cu") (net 14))
 (segment (start 182.25 108.88) (end 136.26 108.88) (width 0.3) (layer "B.Cu") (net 14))
 (segment (start 136.26 108.88) (end 122.73 95.35) (width 0.3) (layer "B.Cu") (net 14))
 (segment (start 186.459999 104.670001) (end 182.25 108.88) (width 0.3) (layer "B.Cu") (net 14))
 (segment (start 180.87 98.9) (end 180.87 98.78) (width 0.3) (layer "B.Cu") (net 14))
 (segment (start 180.87 98.78) (end 182.17 97.48) (width 0.3) (layer "B.Cu") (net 14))
 (segment (start 184.85 97.48) (end 186.459999 99.089999) (width 0.3) (layer "B.Cu") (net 14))
 (segment (start 182.17 97.48) (end 184.85 97.48) (width 0.3) (layer "B.Cu") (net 14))
 (segment (start 186.459999 99.089999) (end 186.459999 104.670001) (width 0.3) (layer "B.Cu") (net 14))
 (segment (start 122.29 89.85) (end 119.114 89.85) (width 0.3) (layer "F.Cu") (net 13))
 (segment (start 119.114 89.85) (end 118.038 90.926) (width 0.3) (layer "F.Cu") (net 13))
 (via (at 122.29 89.85) (size 0.8) (drill 0.4) (layers "F.Cu" "B.Cu") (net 13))
 (segment (start 139.19386 95.685084) (end 140.105082 94.773857) (width 0.3) (layer "B.Cu") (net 13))
 (segment (start 143.074949 97.743725) (end 142.163722 98.654947) (width 0.3) (layer "B.Cu") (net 13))
 (segment (start 139.680817 94.349592) (end 139.680817 94.349593) (width 0.3) (layer "B.Cu") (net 13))
 (segment (start 140.52935 95.198125) (end 140.52935 95.198126) (width 0.3) (layer "B.Cu") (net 13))
 (segment (start 141.739459 98.230683) (end 142.650681 97.319456) (width 0.3) (layer "B.Cu") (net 13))
 (segment (start 140.042393 96.533617) (end 140.953615 95.62239) (width 0.3) (layer "B.Cu") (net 13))
 (segment (start 138.832284 93.501059) (end 138.832284 93.50106) (width 0.3) (layer "B.Cu") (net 13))
 (segment (start 142.226416 96.895191) (end 142.226416 96.895192) (width 0.3) (layer "B.Cu") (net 13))
 (segment (start 138.832284 93.50106) (end 138.588803 93.74454) (width 0.3) (layer "B.Cu") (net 13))
 (segment (start 134.27 89.85) (end 122.29 89.85) (width 0.3) (layer "B.Cu") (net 13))
 (segment (start 141.377883 96.046659) (end 140.466656 96.957881) (width 0.3) (layer "B.Cu") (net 13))
 (segment (start 143.255735 99.259999) (end 143.255734 99.259999) (width 0.3) (layer "B.Cu") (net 13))
 (segment (start 140.890926 97.38215) (end 141.802148 96.470923) (width 0.3) (layer "B.Cu") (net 13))
 (segment (start 143.074949 97.743724) (end 143.074949 97.743725) (width 0.3) (layer "B.Cu") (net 13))
 (segment (start 138.345325 94.83655) (end 138.345327 94.836551) (width 0.3) (layer "B.Cu") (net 13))
 (segment (start 141.377883 96.046658) (end 141.377883 96.046659) (width 0.3) (layer "B.Cu") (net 13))
 (segment (start 139.680817 94.349593) (end 138.76959 95.260815) (width 0.3) (layer "B.Cu") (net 13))
 (segment (start 140.042391 96.533616) (end 140.042393 96.533617) (width 0.3) (layer "B.Cu") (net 13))
 (segment (start 179.85 101.44) (end 179.85 102.62) (width 0.3) (layer "B.Cu") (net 13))
 (segment (start 142.226416 96.895192) (end 141.315189 97.806414) (width 0.3) (layer "B.Cu") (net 13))
 (segment (start 138.164539 93.74454) (end 134.27 89.85) (width 0.3) (layer "B.Cu") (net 13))
 (segment (start 143.255734 99.259999) (end 143.012254 99.50348) (width 0.3) (layer "B.Cu") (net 13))
 (segment (start 140.890924 97.382149) (end 140.890926 97.38215) (width 0.3) (layer "B.Cu") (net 13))
 (segment (start 140.52935 95.198126) (end 139.618123 96.109348) (width 0.3) (layer "B.Cu") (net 13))
 (segment (start 139.193858 95.685083) (end 139.19386 95.685084) (width 0.3) (layer "B.Cu") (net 13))
 (segment (start 151.97 107.55) (end 143.68 99.26) (width 0.3) (layer "B.Cu") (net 13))
 (segment (start 179.85 102.62) (end 174.92 107.55) (width 0.3) (layer "B.Cu") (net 13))
 (segment (start 142.587989 99.079214) (end 143.499214 98.167989) (width 0.3) (layer "B.Cu") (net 13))
 (segment (start 141.739457 98.230682) (end 141.739459 98.230683) (width 0.3) (layer "B.Cu") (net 13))
 (segment (start 142.587989 99.079215) (end 142.587989 99.079214) (width 0.3) (layer "B.Cu") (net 13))
 (segment (start 174.92 107.55) (end 151.97 107.55) (width 0.3) (layer "B.Cu") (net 13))
 (segment (start 138.345327 94.836551) (end 139.256549 93.925324) (width 0.3) (layer "B.Cu") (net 13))
 (arc (start 143.499214 98.167989) (mid 143.587082 97.955857) (end 143.499214 97.743725) (width 0.3) (layer "B.Cu") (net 13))
 (arc (start 138.76959 95.260815) (mid 138.557458 95.348683) (end 138.345326 95.260815) (width 0.3) (layer "B.Cu") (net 13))
 (arc (start 142.58799 99.50348) (mid 142.50012 99.291347) (end 142.587989 99.079215) (width 0.3) (layer "B.Cu") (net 13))
 (arc (start 143.68 99.26) (mid 143.467867 99.17213) (end 143.255735 99.259999) (width 0.3) (layer "B.Cu") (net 13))
 (arc (start 139.256549 93.50106) (mid 139.044417 93.413191) (end 138.832284 93.501059) (width 0.3) (layer "B.Cu") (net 13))
 (arc (start 141.739458 98.654947) (mid 141.65159 98.442816) (end 141.739457 98.230682) (width 0.3) (layer "B.Cu") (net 13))
 (arc (start 141.802148 96.046659) (mid 141.590016 95.95879) (end 141.377883 96.046658) (width 0.3) (layer "B.Cu") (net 13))
 (arc (start 138.345326 95.260815) (mid 138.257458 95.048684) (end 138.345325 94.83655) (width 0.3) (layer "B.Cu") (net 13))
 (arc (start 140.890925 97.806414) (mid 140.803057 97.594283) (end 140.890924 97.382149) (width 0.3) (layer "B.Cu") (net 13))
 (arc (start 141.315189 97.806414) (mid 141.103057 97.894282) (end 140.890925 97.806414) (width 0.3) (layer "B.Cu") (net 13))
 (arc (start 143.012254 99.50348) (mid 142.800122 99.591348) (end 142.58799 99.50348) (width 0.3) (layer "B.Cu") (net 13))
 (arc (start 141.802148 96.470923) (mid 141.890016 96.258791) (end 141.802148 96.046659) (width 0.3) (layer "B.Cu") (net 13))
 (arc (start 140.042392 96.957881) (mid 139.954524 96.74575) (end 140.042391 96.533616) (width 0.3) (layer "B.Cu") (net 13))
 (arc (start 142.163722 98.654947) (mid 141.95159 98.742815) (end 141.739458 98.654947) (width 0.3) (layer "B.Cu") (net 13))
 (arc (start 140.105082 94.349593) (mid 139.89295 94.261724) (end 139.680817 94.349592) (width 0.3) (layer "B.Cu") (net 13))
 (arc (start 142.650681 97.319456) (mid 142.738549 97.107324) (end 142.650681 96.895192) (width 0.3) (layer "B.Cu") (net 13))
 (arc (start 142.650681 96.895192) (mid 142.438549 96.807323) (end 142.226416 96.895191) (width 0.3) (layer "B.Cu") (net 13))
 (arc (start 139.256549 93.925324) (mid 139.344417 93.713192) (end 139.256549 93.50106) (width 0.3) (layer "B.Cu") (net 13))
 (arc (start 140.466656 96.957881) (mid 140.254524 97.045749) (end 140.042392 96.957881) (width 0.3) (layer "B.Cu") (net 13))
 (arc (start 143.499214 97.743725) (mid 143.287082 97.655856) (end 143.074949 97.743724) (width 0.3) (layer "B.Cu") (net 13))
 (arc (start 138.588803 93.74454) (mid 138.376671 93.832408) (end 138.164539 93.74454) (width 0.3) (layer "B.Cu") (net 13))
 (arc (start 139.618123 96.109348) (mid 139.405991 96.197216) (end 139.193859 96.109348) (width 0.3) (layer "B.Cu") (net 13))
 (arc (start 140.105082 94.773857) (mid 140.19295 94.561725) (end 140.105082 94.349593) (width 0.3) (layer "B.Cu") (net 13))
 (arc (start 140.953615 95.198126) (mid 140.741483 95.110257) (end 140.52935 95.198125) (width 0.3) (layer "B.Cu") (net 13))
 (arc (start 139.193859 96.109348) (mid 139.105991 95.897217) (end 139.193858 95.685083) (width 0.3) (layer "B.Cu") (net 13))
 (arc (start 140.953615 95.62239) (mid 141.041483 95.410258) (end 140.953615 95.198126) (width 0.3) (layer "B.Cu") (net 13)))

